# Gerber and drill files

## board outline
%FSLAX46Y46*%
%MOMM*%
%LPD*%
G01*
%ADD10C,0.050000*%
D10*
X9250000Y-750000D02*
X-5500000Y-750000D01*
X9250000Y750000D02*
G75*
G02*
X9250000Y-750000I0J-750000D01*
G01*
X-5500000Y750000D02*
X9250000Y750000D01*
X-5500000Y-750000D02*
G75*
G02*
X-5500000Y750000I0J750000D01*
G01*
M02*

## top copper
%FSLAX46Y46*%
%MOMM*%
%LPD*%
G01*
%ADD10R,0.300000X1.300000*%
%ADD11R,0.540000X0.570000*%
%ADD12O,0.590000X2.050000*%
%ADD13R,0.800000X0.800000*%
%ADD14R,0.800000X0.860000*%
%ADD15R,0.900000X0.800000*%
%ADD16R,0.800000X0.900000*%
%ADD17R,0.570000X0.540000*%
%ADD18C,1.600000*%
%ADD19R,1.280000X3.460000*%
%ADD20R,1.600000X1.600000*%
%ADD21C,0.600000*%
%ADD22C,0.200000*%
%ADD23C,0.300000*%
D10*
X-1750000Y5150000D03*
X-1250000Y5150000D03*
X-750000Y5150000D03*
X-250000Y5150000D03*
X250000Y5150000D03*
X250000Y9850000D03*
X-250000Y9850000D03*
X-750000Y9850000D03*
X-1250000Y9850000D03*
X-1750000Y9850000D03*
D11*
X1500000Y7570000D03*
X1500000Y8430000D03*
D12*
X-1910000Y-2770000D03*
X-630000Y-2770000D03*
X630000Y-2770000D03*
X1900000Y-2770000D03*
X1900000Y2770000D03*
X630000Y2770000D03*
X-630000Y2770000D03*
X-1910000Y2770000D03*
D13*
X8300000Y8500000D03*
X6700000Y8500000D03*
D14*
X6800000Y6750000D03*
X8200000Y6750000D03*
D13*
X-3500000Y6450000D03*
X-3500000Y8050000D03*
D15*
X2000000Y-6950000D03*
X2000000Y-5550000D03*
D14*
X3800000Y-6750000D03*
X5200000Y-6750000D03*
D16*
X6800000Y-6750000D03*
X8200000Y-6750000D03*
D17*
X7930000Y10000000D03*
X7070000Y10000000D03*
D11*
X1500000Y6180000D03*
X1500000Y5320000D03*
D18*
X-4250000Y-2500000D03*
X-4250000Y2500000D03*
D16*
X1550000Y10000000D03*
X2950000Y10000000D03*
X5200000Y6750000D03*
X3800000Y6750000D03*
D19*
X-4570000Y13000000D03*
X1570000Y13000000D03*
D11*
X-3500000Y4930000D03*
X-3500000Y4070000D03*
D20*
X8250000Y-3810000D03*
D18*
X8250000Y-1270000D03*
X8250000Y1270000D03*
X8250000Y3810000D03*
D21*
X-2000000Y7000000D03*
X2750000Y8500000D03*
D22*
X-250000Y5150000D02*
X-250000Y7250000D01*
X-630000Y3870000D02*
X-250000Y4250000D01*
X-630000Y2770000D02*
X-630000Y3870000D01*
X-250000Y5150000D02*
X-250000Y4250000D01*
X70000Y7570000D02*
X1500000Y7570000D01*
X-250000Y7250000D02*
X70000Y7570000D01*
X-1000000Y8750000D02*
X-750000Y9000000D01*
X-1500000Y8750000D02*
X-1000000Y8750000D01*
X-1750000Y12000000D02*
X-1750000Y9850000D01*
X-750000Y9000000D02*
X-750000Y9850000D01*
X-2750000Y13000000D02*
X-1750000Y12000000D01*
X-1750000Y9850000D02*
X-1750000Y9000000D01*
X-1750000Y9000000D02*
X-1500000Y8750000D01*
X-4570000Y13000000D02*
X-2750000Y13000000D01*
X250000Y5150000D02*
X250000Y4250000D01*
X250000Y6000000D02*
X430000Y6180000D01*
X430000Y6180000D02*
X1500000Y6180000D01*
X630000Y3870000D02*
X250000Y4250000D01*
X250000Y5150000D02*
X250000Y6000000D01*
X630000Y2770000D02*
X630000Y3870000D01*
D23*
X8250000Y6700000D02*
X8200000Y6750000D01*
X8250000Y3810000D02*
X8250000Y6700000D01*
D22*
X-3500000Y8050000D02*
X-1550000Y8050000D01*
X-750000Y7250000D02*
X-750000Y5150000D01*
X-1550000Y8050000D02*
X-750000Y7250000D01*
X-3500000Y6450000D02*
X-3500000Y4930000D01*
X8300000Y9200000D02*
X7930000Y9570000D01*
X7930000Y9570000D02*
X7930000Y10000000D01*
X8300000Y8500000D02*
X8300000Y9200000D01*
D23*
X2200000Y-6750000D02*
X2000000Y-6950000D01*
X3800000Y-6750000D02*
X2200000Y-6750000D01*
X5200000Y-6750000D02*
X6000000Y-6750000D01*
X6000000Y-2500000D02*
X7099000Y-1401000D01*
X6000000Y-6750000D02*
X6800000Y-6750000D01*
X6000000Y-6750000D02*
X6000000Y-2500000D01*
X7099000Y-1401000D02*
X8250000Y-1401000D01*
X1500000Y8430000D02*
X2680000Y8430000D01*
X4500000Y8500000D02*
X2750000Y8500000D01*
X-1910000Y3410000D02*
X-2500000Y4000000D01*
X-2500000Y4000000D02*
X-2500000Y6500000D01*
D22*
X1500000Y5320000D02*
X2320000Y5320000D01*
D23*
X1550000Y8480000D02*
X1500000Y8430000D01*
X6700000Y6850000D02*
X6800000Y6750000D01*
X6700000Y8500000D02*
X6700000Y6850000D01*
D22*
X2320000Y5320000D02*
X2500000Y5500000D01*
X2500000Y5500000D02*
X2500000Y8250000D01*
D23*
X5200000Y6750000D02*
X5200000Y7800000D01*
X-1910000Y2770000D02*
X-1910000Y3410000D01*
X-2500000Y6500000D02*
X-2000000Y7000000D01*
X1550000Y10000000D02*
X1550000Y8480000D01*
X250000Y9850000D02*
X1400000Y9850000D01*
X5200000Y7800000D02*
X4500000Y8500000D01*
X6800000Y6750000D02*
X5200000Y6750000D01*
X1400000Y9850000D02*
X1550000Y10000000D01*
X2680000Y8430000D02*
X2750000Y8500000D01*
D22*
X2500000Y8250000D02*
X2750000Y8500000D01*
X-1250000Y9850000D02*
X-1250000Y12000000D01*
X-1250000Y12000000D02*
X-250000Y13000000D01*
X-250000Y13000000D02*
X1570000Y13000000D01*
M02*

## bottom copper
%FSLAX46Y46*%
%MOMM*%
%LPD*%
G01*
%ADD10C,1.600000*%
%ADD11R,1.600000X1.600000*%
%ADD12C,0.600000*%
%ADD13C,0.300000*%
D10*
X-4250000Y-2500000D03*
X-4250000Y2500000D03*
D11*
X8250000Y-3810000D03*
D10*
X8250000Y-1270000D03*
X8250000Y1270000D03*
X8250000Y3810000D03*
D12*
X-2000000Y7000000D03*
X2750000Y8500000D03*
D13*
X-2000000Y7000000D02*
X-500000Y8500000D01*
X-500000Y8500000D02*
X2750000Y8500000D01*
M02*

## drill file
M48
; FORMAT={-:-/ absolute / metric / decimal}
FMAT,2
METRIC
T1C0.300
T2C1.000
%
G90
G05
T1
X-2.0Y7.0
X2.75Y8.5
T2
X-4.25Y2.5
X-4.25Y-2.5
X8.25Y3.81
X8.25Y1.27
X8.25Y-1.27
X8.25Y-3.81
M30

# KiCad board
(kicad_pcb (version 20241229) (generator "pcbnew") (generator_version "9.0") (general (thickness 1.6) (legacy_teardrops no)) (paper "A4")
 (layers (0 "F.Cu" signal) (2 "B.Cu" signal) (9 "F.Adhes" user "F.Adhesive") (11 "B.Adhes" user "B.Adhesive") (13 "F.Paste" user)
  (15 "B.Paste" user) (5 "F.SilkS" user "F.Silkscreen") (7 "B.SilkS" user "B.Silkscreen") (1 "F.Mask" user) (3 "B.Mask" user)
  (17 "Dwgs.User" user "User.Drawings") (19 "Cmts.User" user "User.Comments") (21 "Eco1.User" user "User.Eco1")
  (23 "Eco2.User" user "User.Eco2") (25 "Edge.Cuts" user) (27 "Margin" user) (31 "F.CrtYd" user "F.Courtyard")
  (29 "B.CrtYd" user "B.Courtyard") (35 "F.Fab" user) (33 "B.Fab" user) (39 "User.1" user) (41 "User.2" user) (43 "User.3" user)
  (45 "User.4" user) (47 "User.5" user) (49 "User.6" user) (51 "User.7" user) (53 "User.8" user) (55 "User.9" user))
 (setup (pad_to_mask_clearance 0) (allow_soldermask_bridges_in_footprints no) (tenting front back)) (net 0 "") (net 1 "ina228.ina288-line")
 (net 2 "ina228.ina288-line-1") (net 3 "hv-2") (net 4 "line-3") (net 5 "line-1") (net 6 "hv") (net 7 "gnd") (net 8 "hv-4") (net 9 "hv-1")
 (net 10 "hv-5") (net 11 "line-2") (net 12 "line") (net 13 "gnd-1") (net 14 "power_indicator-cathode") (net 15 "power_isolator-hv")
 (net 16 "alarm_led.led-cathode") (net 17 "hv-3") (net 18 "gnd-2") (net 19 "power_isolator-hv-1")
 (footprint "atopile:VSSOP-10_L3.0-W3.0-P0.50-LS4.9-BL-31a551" (layer "F.Cu") (at -0.75 -7.5)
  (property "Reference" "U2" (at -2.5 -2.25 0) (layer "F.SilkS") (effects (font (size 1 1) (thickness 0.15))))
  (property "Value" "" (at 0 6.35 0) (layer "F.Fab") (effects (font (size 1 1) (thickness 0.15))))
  (pad "1" smd rect (at -1 2.35) (size 0.3 1.3) (layers "F.Cu" "F.Mask" "F.Paste") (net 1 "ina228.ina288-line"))
  (pad "2" smd rect (at -0.5 2.35) (size 0.3 1.3) (layers "F.Cu" "F.Mask" "F.Paste") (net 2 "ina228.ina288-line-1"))
  (pad "3" smd rect (at 0 2.35) (size 0.3 1.3) (layers "F.Cu" "F.Mask" "F.Paste") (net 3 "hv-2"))
  (pad "4" smd rect (at 0.5 2.35) (size 0.3 1.3) (layers "F.Cu" "F.Mask" "F.Paste") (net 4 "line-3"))
  (pad "5" smd rect (at 1 2.35) (size 0.3 1.3) (layers "F.Cu" "F.Mask" "F.Paste") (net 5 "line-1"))
  (pad "6" smd rect (at 1 -2.35) (size 0.3 1.3) (layers "F.Cu" "F.Mask" "F.Paste") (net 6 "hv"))
  (pad "7" smd rect (at 0.5 -2.35) (size 0.3 1.3) (layers "F.Cu" "F.Mask" "F.Paste") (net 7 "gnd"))
  (pad "8" smd rect (at 0 -2.35) (size 0.3 1.3) (layers "F.Cu" "F.Mask" "F.Paste") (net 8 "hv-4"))
  (pad "9" smd rect (at -0.5 -2.35) (size 0.3 1.3) (layers "F.Cu" "F.Mask" "F.Paste") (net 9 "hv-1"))
  (pad "10" smd rect (at -1 -2.35) (size 0.3 1.3) (layers "F.Cu" "F.Mask" "F.Paste") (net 8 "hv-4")))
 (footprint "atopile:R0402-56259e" (layer "F.Cu") (at 1.5 -8 90)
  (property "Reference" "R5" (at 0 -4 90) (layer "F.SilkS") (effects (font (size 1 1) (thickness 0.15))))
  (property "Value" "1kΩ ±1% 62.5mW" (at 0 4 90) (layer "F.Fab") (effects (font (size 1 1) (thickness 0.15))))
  (pad "1" smd rect (at -0.43 0 90) (size 0.57 0.54) (layers "F.Cu" "F.Mask" "F.Paste") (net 4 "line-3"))
  (pad "2" smd rect (at 0.43 0 90) (size 0.57 0.54) (layers "F.Cu" "F.Mask" "F.Paste") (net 6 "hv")))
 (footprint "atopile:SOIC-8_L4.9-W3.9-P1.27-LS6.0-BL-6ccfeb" (layer "F.Cu") (at 0 0)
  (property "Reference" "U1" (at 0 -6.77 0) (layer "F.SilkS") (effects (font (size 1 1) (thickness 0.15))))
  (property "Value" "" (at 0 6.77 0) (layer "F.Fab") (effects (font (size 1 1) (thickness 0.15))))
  (pad "1" smd oval (at -1.91 2.77) (size 0.59 2.05) (layers "F.Cu" "F.Mask" "F.Paste") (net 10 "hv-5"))
  (pad "2" smd oval (at -0.63 2.77) (size 0.59 2.05) (layers "F.Cu" "F.Mask" "F.Paste") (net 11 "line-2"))
  (pad "3" smd oval (at 0.63 2.77) (size 0.59 2.05) (layers "F.Cu" "F.Mask" "F.Paste") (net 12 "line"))
  (pad "4" smd oval (at 1.9 2.77) (size 0.59 2.05) (layers "F.Cu" "F.Mask" "F.Paste") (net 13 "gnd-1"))
  (pad "5" smd oval (at 1.9 -2.77) (size 0.59 2.05) (layers "F.Cu" "F.Mask" "F.Paste") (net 7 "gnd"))
  (pad "6" smd oval (at 0.63 -2.77) (size 0.59 2.05) (layers "F.Cu" "F.Mask" "F.Paste") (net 5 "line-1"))
  (pad "7" smd oval (at -0.63 -2.77) (size 0.59 2.05) (layers "F.Cu" "F.Mask" "F.Paste") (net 4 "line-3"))
  (pad "8" smd oval (at -1.91 -2.77) (size 0.59 2.05) (layers "F.Cu" "F.Mask" "F.Paste") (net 6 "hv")))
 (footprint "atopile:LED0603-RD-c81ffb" (layer "F.Cu") (at 7.5 -8.5 180)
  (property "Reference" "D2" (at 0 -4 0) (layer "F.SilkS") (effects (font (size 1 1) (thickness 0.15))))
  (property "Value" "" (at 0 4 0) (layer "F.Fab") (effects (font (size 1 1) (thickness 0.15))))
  (pad "1" smd rect (at -0.8 0 270) (size 0.8 0.8) (layers "F.Cu" "F.Mask" "F.Paste") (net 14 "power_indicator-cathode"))
  (pad "2" smd rect (at 0.8 0 270) (size 0.8 0.8) (layers "F.Cu" "F.Mask" "F.Paste") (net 6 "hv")))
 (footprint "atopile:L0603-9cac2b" (layer "F.Cu") (at 7.5 -6.75)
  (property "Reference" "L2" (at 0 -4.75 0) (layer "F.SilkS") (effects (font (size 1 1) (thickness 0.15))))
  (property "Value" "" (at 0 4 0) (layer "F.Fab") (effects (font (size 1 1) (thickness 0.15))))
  (pad "1" smd rect (at -0.7 0 180) (size 0.8 0.86) (layers "F.Cu" "F.Mask" "F.Paste") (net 6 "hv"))
  (pad "2" smd rect (at 0.7 0 180) (size 0.8 0.86) (layers "F.Cu" "F.Mask" "F.Paste") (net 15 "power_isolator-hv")))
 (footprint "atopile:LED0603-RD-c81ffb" (layer "F.Cu") (at -3.5 -7.25 90)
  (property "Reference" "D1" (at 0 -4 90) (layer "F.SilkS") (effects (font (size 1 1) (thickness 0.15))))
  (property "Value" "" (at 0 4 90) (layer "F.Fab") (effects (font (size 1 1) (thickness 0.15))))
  (pad "1" smd rect (at -0.8 0 180) (size 0.8 0.8) (layers "F.Cu" "F.Mask" "F.Paste") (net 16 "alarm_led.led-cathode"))
  (pad "2" smd rect (at 0.8 0 180) (size 0.8 0.8) (layers "F.Cu" "F.Mask" "F.Paste") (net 3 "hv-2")))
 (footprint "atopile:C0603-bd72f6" (layer "F.Cu") (at 2 6.25 90)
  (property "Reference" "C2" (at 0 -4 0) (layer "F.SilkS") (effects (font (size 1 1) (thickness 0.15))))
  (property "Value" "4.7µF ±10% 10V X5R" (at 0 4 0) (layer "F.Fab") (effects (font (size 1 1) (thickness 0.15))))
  (pad "1" smd rect (at -0.7 0 90) (size 0.8 0.9) (layers "F.Cu" "F.Mask" "F.Paste") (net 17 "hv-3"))
  (pad "2" smd rect (at 0.7 0 90) (size 0.8 0.9) (layers "F.Cu" "F.Mask" "F.Paste") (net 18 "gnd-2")))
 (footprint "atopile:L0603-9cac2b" (layer "F.Cu") (at 4.5 6.75)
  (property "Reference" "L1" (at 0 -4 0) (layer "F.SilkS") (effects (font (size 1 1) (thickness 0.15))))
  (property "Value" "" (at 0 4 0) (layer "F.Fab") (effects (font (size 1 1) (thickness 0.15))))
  (pad "1" smd rect (at -0.7 0 180) (size 0.8 0.86) (layers "F.Cu" "F.Mask" "F.Paste") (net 17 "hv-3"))
  (pad "2" smd rect (at 0.7 0 180) (size 0.8 0.86) (layers "F.Cu" "F.Mask" "F.Paste") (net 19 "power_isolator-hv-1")))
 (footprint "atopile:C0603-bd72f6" (layer "F.Cu") (at 7.5 6.75)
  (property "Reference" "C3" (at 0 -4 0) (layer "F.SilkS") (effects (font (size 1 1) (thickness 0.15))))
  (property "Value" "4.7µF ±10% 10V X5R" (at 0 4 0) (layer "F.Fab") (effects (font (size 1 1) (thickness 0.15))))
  (pad "1" smd rect (at -0.7 0) (size 0.8 0.9) (layers "F.Cu" "F.Mask" "F.Paste") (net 19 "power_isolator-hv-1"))
  (pad "2" smd rect (at 0.7 0) (size 0.8 0.9) (layers "F.Cu" "F.Mask" "F.Paste") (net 18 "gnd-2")))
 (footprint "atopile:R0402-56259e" (layer "F.Cu") (at 7.5 -10 180)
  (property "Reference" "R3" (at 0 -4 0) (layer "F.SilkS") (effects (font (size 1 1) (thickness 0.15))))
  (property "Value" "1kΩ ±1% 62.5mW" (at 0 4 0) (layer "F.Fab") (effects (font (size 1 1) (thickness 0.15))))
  (pad "1" smd rect (at -0.43 0 180) (size 0.57 0.54) (layers "F.Cu" "F.Mask" "F.Paste") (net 14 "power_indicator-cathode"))
  (pad "2" smd rect (at 0.43 0 180) (size 0.57 0.54) (layers "F.Cu" "F.Mask" "F.Paste") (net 7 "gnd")))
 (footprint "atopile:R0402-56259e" (layer "F.Cu") (at 1.5 -5.75 -90)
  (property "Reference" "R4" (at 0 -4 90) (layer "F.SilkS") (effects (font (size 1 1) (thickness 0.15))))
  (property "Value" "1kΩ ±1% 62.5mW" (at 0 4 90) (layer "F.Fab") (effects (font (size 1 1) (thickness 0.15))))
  (pad "1" smd rect (at -0.43 0 270) (size 0.57 0.54) (layers "F.Cu" "F.Mask" "F.Paste") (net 5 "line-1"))
  (pad "2" smd rect (at 0.43 0 270) (size 0.57 0.54) (layers "F.Cu" "F.Mask" "F.Paste") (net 6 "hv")))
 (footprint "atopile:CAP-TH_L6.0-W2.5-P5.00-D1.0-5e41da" (layer "F.Cu") (at -4.25 0 90)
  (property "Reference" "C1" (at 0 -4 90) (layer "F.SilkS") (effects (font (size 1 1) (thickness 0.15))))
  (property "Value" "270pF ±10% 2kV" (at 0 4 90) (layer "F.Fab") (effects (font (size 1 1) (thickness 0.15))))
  (pad "1" thru_hole circle (at -2.5 0 90) (size 1.6 1.6) (drill 0.999998) (layers "*.Cu" "*.Mask") (remove_unused_layers no)
   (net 18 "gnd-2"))
  (pad "2" thru_hole circle (at 2.5 0 90) (size 1.6 1.6) (drill 0.999998) (layers "*.Cu" "*.Mask") (remove_unused_layers no) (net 7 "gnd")))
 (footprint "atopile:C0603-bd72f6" (layer "F.Cu") (at 2.25 -10)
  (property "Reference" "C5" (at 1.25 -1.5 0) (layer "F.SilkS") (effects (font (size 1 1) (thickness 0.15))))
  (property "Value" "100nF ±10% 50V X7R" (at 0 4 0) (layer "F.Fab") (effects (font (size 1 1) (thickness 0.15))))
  (pad "1" smd rect (at -0.7 0) (size 0.8 0.9) (layers "F.Cu" "F.Mask" "F.Paste") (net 6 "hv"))
  (pad "2" smd rect (at 0.7 0) (size 0.8 0.9) (layers "F.Cu" "F.Mask" "F.Paste") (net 7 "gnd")))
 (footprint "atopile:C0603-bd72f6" (layer "F.Cu") (at 4.5 -6.75 180)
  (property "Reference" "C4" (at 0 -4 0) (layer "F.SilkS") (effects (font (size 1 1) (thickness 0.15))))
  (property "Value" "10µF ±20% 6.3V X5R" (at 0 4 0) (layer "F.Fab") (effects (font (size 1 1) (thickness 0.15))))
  (pad "1" smd rect (at -0.7 0 180) (size 0.8 0.9) (layers "F.Cu" "F.Mask" "F.Paste") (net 6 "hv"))
  (pad "2" smd rect (at 0.7 0 180) (size 0.8 0.9) (layers "F.Cu" "F.Mask" "F.Paste") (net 7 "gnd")))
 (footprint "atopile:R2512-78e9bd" (layer "F.Cu") (at -1.5 -13)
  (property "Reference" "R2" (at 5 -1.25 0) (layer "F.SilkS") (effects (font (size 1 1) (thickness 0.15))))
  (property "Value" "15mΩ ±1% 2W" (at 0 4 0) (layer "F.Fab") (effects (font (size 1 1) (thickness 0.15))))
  (pad "1" smd rect (at -3.07 0) (size 1.28 3.46) (layers "F.Cu" "F.Mask" "F.Paste") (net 8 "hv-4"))
  (pad "2" smd rect (at 3.07 0) (size 1.28 3.46) (layers "F.Cu" "F.Mask" "F.Paste") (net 9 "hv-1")))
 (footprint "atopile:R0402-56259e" (layer "F.Cu") (at -3.5 -4.5 -90)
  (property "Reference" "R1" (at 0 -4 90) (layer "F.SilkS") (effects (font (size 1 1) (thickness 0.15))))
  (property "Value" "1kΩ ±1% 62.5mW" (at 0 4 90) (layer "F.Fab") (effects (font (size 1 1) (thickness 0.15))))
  (pad "1" smd rect (at -0.43 0 270) (size 0.57 0.54) (layers "F.Cu" "F.Mask" "F.Paste") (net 16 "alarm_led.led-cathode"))
  (pad "2" smd rect (at 0.43 0 270) (size 0.57 0.54) (layers "F.Cu" "F.Mask" "F.Paste") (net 7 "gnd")))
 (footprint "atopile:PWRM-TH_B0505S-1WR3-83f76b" (layer "F.Cu") (at 8.25 0 90)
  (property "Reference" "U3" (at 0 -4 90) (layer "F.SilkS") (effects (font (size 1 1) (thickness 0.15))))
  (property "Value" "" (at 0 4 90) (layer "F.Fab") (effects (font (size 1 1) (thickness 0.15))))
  (pad "1" thru_hole rect (at -3.81 0 90) (size 1.6 1.6) (drill 0.999998) (layers "*.Cu" "*.Mask") (remove_unused_layers no)
   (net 18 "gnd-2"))
  (pad "2" thru_hole circle (at -1.27 0 90) (size 1.6 1.6) (drill 0.999998) (layers "*.Cu" "*.Mask") (remove_unused_layers no)
   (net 19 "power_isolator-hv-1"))
  (pad "3" thru_hole circle (at 1.27 0 90) (size 1.6 1.6) (drill 0.999998) (layers "*.Cu" "*.Mask") (remove_unused_layers no) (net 7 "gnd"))
  (pad "4" thru_hole circle (at 3.81 0 90) (size 1.6 1.6) (drill 0.999998) (layers "*.Cu" "*.Mask") (remove_unused_layers no)
   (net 15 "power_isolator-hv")))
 (gr_line (start 9.25 0.75) (end -5.5 0.75) (stroke (width 0.05) (type default)) (layer "Edge.Cuts"))
 (gr_arc (start 9.25 -0.75) (mid 10 0) (end 9.25 0.75) (stroke (width 0.05) (type default)) (layer "Edge.Cuts"))
 (gr_line (start -5.5 -0.75) (end 9.25 -0.75) (stroke (width 0.05) (type default)) (layer "Edge.Cuts"))
 (gr_arc (start -5.5 0.75) (mid -6.25 0) (end -5.5 -0.75) (stroke (width 0.05) (type default)) (layer "Edge.Cuts"))
 (segment (start -0.25 -5.15) (end -0.25 -7.25) (width 0.2) (layer "F.Cu") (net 4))
 (segment (start -0.63 -3.87) (end -0.25 -4.25) (width 0.2) (layer "F.Cu") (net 4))
 (segment (start -0.63 -2.77) (end -0.63 -3.87) (width 0.2) (layer "F.Cu") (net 4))
 (segment (start -0.25 -5.15) (end -0.25 -4.25) (width 0.2) (layer "F.Cu") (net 4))
 (segment (start 0.07 -7.57) (end 1.5 -7.57) (width 0.2) (layer "F.Cu") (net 4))
 (segment (start -0.25 -7.25) (end 0.07 -7.57) (width 0.2) (layer "F.Cu") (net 4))
 (segment (start -1 -8.75) (end -0.75 -9) (width 0.2) (layer "F.Cu") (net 8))
 (segment (start -1.5 -8.75) (end -1 -8.75) (width 0.2) (layer "F.Cu") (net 8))
 (segment (start -1.75 -12) (end -1.75 -9.85) (width 0.2) (layer "F.Cu") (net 8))
 (segment (start -0.75 -9) (end -0.75 -9.85) (width 0.2) (layer "F.Cu") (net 8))
 (segment (start -2.75 -13) (end -1.75 -12) (width 0.2) (layer "F.Cu") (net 8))
 (segment (start -1.75 -9.85) (end -1.75 -9) (width 0.2) (layer "F.Cu") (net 8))
 (segment (start -1.75 -9) (end -1.5 -8.75) (width 0.2) (layer "F.Cu") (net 8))
 (segment (start -4.57 -13) (end -2.75 -13) (width 0.2) (layer "F.Cu") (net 8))
 (segment (start 0.25 -5.15) (end 0.25 -4.25) (width 0.2) (layer "F.Cu") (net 5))
 (segment (start 0.25 -6) (end 0.43 -6.18) (width 0.2) (layer "F.Cu") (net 5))
 (segment (start 0.43 -6.18) (end 1.5 -6.18) (width 0.2) (layer "F.Cu") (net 5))
 (segment (start 0.63 -3.87) (end 0.25 -4.25) (width 0.2) (layer "F.Cu") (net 5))
 (segment (start 0.25 -5.15) (end 0.25 -6) (width 0.2) (layer "F.Cu") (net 5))
 (segment (start 0.63 -2.77) (end 0.63 -3.87) (width 0.2) (layer "F.Cu") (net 5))
 (segment (start 8.25 -6.7) (end 8.2 -6.75) (width 0.3) (layer "F.Cu") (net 15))
 (segment (start 8.25 -3.81) (end 8.25 -6.7) (width 0.3) (layer "F.Cu") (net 15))
 (segment (start -3.5 -8.05) (end -1.55 -8.05) (width 0.2) (layer "F.Cu") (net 3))
 (segment (start -0.75 -7.25) (end -0.75 -5.15) (width 0.2) (layer "F.Cu") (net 3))
 (segment (start -1.55 -8.05) (end -0.75 -7.25) (width 0.2) (layer "F.Cu") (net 3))
 (segment (start -3.5 -6.45) (end -3.5 -4.93) (width 0.2) (layer "F.Cu") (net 16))
 (segment (start 8.3 -9.2) (end 7.93 -9.57) (width 0.2) (layer "F.Cu") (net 14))
 (segment (start 7.93 -9.57) (end 7.93 -10) (width 0.2) (layer "F.Cu") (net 14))
 (segment (start 8.3 -8.5) (end 8.3 -9.2) (width 0.2) (layer "F.Cu") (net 14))
 (segment (start 2.2 6.75) (end 2 6.95) (width 0.3) (layer "F.Cu") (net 17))
 (segment (start 3.8 6.75) (end 2.2 6.75) (width 0.3) (layer "F.Cu") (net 17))
 (segment (start 5.2 6.75) (end 6 6.75) (width 0.3) (layer "F.Cu") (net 19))
 (segment (start 6 2.5) (end 7.099 1.401) (width 0.3) (layer "F.Cu") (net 19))
 (segment (start 6 6.75) (end 6.8 6.75) (width 0.3) (layer "F.Cu") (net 19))
 (segment (start 6 6.75) (end 6 2.5) (width 0.3) (layer "F.Cu") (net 19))
 (segment (start 7.099 1.401) (end 8.25 1.401) (width 0.3) (layer "F.Cu") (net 19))
 (segment (start 1.5 -8.43) (end 2.68 -8.43) (width 0.3) (layer "F.Cu") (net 6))
 (segment (start 4.5 -8.5) (end 2.75 -8.5) (width 0.3) (layer "F.Cu") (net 6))
 (segment (start -1.91 -3.41) (end -2.5 -4) (width 0.3) (layer "F.Cu") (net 6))
 (segment (start -2.5 -4) (end -2.5 -6.5) (width 0.3) (layer "F.Cu") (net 6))
 (segment (start 1.5 -5.32) (end 2.32 -5.32) (width 0.2) (layer "F.Cu") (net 6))
 (segment (start 1.55 -8.48) (end 1.5 -8.43) (width 0.3) (layer "F.Cu") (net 6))
 (segment (start 6.7 -6.85) (end 6.8 -6.75) (width 0.3) (layer "F.Cu") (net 6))
 (segment (start 6.7 -8.5) (end 6.7 -6.85) (width 0.3) (layer "F.Cu") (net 6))
 (segment (start 2.32 -5.32) (end 2.5 -5.5) (width 0.2) (layer "F.Cu") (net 6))
 (segment (start 2.5 -5.5) (end 2.5 -8.25) (width 0.2) (layer "F.Cu") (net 6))
 (segment (start 5.2 -6.75) (end 5.2 -7.8) (width 0.3) (layer "F.Cu") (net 6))
 (segment (start -1.91 -2.77) (end -1.91 -3.41) (width 0.3) (layer "F.Cu") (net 6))
 (segment (start -2.5 -6.5) (end -2 -7) (width 0.3) (layer "F.Cu") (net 6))
 (segment (start 1.55 -10) (end 1.55 -8.48) (width 0.3) (layer "F.Cu") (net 6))
 (segment (start 0.25 -9.85) (end 1.4 -9.85) (width 0.3) (layer "F.Cu") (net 6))
 (segment (start 5.2 -7.8) (end 4.5 -8.5) (width 0.3) (layer "F.Cu") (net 6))
 (segment (start 6.8 -6.75) (end 5.2 -6.75) (width 0.3) (layer "F.Cu") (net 6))
 (segment (start 1.4 -9.85) (end 1.55 -10) (width 0.3) (layer "F.Cu") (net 6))
 (segment (start 2.68 -8.43) (end 2.75 -8.5) (width 0.3) (layer "F.Cu") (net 6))
 (segment (start 2.5 -8.25) (end 2.75 -8.5) (width 0.2) (layer "F.Cu") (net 6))
 (via (at -2 -7) (size 0.6) (drill 0.3) (layers "F.Cu" "B.Cu") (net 6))
 (via (at 2.75 -8.5) (size 0.6) (drill 0.3) (layers "F.Cu" "B.Cu") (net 6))
 (segment (start -2 -7) (end -0.5 -8.5) (width 0.3) (layer "B.Cu") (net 6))
 (segment (start -0.5 -8.5) (end 2.75 -8.5) (width 0.3) (layer "B.Cu") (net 6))
 (segment (start -1.25 -9.85) (end -1.25 -12) (width 0.2) (layer "F.Cu") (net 9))
 (segment (start -1.25 -12) (end -0.25 -13) (width 0.2) (layer "F.Cu") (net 9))
 (segment (start -0.25 -13) (end 1.57 -13) (width 0.2) (layer "F.Cu") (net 9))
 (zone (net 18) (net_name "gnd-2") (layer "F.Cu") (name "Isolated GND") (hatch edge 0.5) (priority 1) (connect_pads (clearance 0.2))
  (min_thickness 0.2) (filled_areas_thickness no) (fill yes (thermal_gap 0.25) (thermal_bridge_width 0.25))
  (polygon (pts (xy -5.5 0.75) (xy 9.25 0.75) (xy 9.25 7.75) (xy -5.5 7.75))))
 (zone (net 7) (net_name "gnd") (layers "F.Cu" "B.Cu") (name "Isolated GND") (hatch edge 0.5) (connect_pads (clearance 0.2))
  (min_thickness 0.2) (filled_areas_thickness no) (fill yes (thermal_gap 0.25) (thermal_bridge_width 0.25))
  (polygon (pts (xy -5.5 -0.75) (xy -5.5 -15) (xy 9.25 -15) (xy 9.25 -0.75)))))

